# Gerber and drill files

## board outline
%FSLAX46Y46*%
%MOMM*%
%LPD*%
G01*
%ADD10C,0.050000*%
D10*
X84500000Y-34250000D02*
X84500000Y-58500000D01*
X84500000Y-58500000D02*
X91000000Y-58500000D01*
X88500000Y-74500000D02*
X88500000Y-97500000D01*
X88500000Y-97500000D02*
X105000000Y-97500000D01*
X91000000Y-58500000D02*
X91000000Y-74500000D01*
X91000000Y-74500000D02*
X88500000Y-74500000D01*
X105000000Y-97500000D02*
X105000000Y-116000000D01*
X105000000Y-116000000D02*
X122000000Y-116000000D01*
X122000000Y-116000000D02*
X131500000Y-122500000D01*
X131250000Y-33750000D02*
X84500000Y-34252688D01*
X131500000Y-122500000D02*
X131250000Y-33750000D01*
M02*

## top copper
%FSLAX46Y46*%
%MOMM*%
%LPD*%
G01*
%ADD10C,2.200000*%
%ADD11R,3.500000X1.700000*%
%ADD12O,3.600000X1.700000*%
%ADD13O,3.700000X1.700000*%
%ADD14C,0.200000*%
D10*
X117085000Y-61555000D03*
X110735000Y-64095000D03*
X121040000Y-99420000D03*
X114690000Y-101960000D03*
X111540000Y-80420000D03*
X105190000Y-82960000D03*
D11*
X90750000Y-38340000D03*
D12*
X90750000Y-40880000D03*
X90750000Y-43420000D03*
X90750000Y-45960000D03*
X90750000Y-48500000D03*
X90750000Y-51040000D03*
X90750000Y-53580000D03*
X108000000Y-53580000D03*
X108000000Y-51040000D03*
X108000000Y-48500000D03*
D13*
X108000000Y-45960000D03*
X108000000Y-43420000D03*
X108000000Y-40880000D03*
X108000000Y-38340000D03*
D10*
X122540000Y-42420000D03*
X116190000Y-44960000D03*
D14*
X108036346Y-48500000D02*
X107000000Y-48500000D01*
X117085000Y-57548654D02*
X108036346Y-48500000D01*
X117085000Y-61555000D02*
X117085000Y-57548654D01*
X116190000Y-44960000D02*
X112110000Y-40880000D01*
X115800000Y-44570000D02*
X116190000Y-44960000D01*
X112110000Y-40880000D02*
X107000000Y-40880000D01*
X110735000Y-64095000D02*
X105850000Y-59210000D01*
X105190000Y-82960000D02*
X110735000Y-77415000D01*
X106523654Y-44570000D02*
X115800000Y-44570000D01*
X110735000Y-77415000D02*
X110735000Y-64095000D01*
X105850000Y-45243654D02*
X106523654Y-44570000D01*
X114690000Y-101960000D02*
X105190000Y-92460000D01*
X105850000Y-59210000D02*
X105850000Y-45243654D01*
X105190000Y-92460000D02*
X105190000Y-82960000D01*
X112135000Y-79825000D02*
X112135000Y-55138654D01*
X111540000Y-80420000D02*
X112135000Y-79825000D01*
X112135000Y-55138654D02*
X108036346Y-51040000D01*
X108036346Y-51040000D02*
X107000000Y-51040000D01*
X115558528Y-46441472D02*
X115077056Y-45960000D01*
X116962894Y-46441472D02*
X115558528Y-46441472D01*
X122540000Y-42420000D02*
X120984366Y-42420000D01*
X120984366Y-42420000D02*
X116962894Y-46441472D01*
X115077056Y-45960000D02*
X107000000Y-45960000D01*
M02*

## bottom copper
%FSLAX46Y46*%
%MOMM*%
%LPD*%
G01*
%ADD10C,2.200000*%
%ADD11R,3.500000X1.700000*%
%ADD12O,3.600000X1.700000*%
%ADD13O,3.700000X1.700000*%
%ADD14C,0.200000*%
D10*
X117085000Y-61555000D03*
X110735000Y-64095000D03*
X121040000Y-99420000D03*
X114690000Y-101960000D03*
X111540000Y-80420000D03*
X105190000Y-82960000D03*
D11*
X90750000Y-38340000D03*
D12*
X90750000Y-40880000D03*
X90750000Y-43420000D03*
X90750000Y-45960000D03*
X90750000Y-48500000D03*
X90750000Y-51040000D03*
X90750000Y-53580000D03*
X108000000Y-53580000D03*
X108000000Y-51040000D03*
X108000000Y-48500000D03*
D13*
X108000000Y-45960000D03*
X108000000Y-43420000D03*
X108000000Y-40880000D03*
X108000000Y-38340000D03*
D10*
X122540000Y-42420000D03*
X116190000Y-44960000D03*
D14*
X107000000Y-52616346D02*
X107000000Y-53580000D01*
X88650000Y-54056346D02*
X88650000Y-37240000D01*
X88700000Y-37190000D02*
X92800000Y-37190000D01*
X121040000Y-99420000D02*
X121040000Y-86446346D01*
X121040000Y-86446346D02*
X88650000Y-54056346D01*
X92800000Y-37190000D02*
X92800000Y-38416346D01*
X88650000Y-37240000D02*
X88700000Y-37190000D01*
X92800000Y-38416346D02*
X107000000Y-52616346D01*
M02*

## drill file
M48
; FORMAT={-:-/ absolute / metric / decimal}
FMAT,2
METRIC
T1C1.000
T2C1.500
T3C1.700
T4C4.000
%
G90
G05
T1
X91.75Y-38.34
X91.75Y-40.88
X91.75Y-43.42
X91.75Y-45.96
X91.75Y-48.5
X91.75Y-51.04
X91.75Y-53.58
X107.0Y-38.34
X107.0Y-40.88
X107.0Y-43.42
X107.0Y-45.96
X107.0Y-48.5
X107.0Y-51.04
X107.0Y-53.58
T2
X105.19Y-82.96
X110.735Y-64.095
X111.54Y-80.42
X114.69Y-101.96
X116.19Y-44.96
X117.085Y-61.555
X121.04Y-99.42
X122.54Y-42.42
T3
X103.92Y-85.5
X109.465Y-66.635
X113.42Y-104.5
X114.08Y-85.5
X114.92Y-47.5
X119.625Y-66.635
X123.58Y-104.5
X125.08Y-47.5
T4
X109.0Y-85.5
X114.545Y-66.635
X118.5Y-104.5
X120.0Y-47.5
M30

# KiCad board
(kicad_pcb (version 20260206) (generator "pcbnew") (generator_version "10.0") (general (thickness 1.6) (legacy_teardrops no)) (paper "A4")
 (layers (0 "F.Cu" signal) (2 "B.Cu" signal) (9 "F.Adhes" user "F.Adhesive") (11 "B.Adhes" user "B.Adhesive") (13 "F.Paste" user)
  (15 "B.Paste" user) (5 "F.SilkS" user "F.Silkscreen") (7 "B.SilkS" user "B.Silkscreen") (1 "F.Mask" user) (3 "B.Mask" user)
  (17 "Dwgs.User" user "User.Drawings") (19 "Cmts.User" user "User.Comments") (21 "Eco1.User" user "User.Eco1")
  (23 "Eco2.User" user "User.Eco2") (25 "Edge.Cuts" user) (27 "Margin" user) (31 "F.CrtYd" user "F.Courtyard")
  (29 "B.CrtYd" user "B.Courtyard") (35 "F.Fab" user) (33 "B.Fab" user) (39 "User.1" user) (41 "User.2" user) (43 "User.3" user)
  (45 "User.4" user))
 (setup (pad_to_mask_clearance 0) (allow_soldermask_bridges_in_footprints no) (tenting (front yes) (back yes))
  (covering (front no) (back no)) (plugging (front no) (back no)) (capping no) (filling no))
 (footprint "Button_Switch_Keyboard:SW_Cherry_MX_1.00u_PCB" (layer "F.Cu") (at 117.085 61.555)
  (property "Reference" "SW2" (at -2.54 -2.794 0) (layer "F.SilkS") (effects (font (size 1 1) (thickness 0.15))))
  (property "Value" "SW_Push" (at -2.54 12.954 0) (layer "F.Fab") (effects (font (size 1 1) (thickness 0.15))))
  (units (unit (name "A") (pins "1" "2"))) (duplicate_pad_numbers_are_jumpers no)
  (pad "" np_thru_hole circle (at -7.62 5.08) (size 1.7 1.7) (drill 1.7) (layers "*.Cu" "*.Mask"))
  (pad "" np_thru_hole circle (at -2.54 5.08) (size 4 4) (drill 4) (layers "*.Cu" "*.Mask"))
  (pad "" np_thru_hole circle (at 2.54 5.08) (size 1.7 1.7) (drill 1.7) (layers "*.Cu" "*.Mask"))
  (pad "1" thru_hole circle (at 0 0) (size 2.2 2.2) (drill 1.5) (layers "*.Cu" "*.Mask") (remove_unused_layers no)
   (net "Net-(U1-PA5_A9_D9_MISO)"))
  (pad "2" thru_hole circle (at -6.35 2.54) (size 2.2 2.2) (drill 1.5) (layers "*.Cu" "*.Mask") (remove_unused_layers no) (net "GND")))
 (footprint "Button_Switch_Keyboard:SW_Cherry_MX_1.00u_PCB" (layer "F.Cu") (at 121.04 99.42)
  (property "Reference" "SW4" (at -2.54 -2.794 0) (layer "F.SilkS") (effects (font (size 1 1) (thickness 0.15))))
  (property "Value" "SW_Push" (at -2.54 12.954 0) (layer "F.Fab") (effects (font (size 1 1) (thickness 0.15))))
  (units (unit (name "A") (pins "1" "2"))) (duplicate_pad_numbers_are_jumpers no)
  (pad "" np_thru_hole circle (at -7.62 5.08) (size 1.7 1.7) (drill 1.7) (layers "*.Cu" "*.Mask"))
  (pad "" np_thru_hole circle (at -2.54 5.08) (size 4 4) (drill 4) (layers "*.Cu" "*.Mask"))
  (pad "" np_thru_hole circle (at 2.54 5.08) (size 1.7 1.7) (drill 1.7) (layers "*.Cu" "*.Mask"))
  (pad "1" thru_hole circle (at 0 0) (size 2.2 2.2) (drill 1.5) (layers "*.Cu" "*.Mask") (remove_unused_layers no)
   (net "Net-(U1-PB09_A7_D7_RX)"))
  (pad "2" thru_hole circle (at -6.35 2.54) (size 2.2 2.2) (drill 1.5) (layers "*.Cu" "*.Mask") (remove_unused_layers no) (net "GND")))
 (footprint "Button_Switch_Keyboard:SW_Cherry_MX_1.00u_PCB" (layer "F.Cu") (at 111.54 80.42)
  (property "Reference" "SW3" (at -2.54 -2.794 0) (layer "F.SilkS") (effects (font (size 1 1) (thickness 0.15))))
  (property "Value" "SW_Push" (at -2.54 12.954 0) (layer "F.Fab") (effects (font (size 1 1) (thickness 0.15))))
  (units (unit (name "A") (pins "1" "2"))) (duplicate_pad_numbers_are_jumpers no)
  (pad "" np_thru_hole circle (at -7.62 5.08) (size 1.7 1.7) (drill 1.7) (layers "*.Cu" "*.Mask"))
  (pad "" np_thru_hole circle (at -2.54 5.08) (size 4 4) (drill 4) (layers "*.Cu" "*.Mask"))
  (pad "" np_thru_hole circle (at 2.54 5.08) (size 1.7 1.7) (drill 1.7) (layers "*.Cu" "*.Mask"))
  (pad "1" thru_hole circle (at 0 0) (size 2.2 2.2) (drill 1.5) (layers "*.Cu" "*.Mask") (remove_unused_layers no)
   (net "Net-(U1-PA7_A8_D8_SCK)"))
  (pad "2" thru_hole circle (at -6.35 2.54) (size 2.2 2.2) (drill 1.5) (layers "*.Cu" "*.Mask") (remove_unused_layers no) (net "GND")))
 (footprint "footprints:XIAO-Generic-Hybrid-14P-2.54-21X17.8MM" (layer "F.Cu") (at 99.375 45.96)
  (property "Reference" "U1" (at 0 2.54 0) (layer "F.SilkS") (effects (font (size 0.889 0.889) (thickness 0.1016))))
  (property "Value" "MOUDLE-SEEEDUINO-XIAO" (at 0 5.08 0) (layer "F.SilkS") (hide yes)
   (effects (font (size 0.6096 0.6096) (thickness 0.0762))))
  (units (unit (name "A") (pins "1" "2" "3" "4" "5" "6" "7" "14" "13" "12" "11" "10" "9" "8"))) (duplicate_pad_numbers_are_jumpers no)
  (pad "1" thru_hole rect (at -7.625 -7.62) (size 3.5 1.7) (drill 1 (offset -1 0)) (layers "*.Cu" "*.Mask") (remove_unused_layers no)
   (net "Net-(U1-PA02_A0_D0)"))
  (pad "2" thru_hole oval (at -7.625 -5.08) (size 3.6 1.7) (drill 1 (offset -1 0)) (layers "*.Cu" "*.Mask") (remove_unused_layers no)
   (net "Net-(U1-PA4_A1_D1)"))
  (pad "3" thru_hole oval (at -7.625 -2.54) (size 3.6 1.7) (drill 1 (offset -1 0)) (layers "*.Cu" "*.Mask") (remove_unused_layers no)
   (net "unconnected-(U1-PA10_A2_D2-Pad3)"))
  (pad "4" thru_hole oval (at -7.625 0) (size 3.6 1.7) (drill 1 (offset -1 0)) (layers "*.Cu" "*.Mask") (remove_unused_layers no)
   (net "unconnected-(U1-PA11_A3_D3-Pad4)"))
  (pad "5" thru_hole oval (at -7.625 2.54) (size 3.6 1.7) (drill 1 (offset -1 0)) (layers "*.Cu" "*.Mask") (remove_unused_layers no)
   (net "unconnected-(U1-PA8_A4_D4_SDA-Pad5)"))
  (pad "6" thru_hole oval (at -7.625 5.08 180) (size 3.6 1.7) (drill 1 (offset 1 0)) (layers "*.Cu" "*.Mask") (remove_unused_layers no)
   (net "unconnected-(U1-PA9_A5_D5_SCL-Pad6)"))
  (pad "7" thru_hole oval (at -7.625 7.62) (size 3.6 1.7) (drill 1 (offset -1 0)) (layers "*.Cu" "*.Mask") (remove_unused_layers no)
   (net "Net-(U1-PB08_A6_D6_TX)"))
  (pad "8" thru_hole oval (at 7.625 7.62) (size 3.6 1.7) (drill 1 (offset 1 0)) (layers "*.Cu" "*.Mask") (remove_unused_layers no)
   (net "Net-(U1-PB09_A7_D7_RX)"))
  (pad "9" thru_hole oval (at 7.625 5.08) (size 3.6 1.7) (drill 1 (offset 1 0)) (layers "*.Cu" "*.Mask") (remove_unused_layers no)
   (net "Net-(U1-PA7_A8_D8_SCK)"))
  (pad "10" thru_hole oval (at 7.625 2.54) (size 3.6 1.7) (drill 1 (offset 1 0)) (layers "*.Cu" "*.Mask") (remove_unused_layers no)
   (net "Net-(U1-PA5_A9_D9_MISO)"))
  (pad "11" thru_hole oval (at 7.625 0) (size 3.7 1.7) (drill 1 (offset 1 0)) (layers "*.Cu" "*.Mask") (remove_unused_layers no)
   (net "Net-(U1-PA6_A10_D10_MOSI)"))
  (pad "12" thru_hole oval (at 7.625 -2.54) (size 3.7 1.7) (drill 1 (offset 1 0)) (layers "*.Cu" "*.Mask") (remove_unused_layers no)
   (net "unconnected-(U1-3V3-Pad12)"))
  (pad "13" thru_hole oval (at 7.625 -5.08) (size 3.7 1.7) (drill 1 (offset 1 0)) (layers "*.Cu" "*.Mask") (remove_unused_layers no)
   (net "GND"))
  (pad "14" thru_hole oval (at 7.625 -7.62) (size 3.7 1.7) (drill 1 (offset 1 0)) (layers "*.Cu" "*.Mask") (remove_unused_layers no)
   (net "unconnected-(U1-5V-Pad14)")))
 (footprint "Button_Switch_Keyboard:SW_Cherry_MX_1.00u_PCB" (layer "F.Cu") (at 122.54 42.42)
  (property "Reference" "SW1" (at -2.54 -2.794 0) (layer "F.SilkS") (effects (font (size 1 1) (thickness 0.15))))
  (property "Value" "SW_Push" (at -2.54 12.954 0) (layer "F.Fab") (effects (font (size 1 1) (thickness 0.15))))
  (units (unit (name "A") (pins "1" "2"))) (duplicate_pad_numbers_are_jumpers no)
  (pad "" np_thru_hole circle (at -7.62 5.08) (size 1.7 1.7) (drill 1.7) (layers "*.Cu" "*.Mask"))
  (pad "" np_thru_hole circle (at -2.54 5.08) (size 4 4) (drill 4) (layers "*.Cu" "*.Mask"))
  (pad "" np_thru_hole circle (at 2.54 5.08) (size 1.7 1.7) (drill 1.7) (layers "*.Cu" "*.Mask"))
  (pad "1" thru_hole circle (at 0 0) (size 2.2 2.2) (drill 1.5) (layers "*.Cu" "*.Mask") (remove_unused_layers no)
   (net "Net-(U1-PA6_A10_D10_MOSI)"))
  (pad "2" thru_hole circle (at -6.35 2.54) (size 2.2 2.2) (drill 1.5) (layers "*.Cu" "*.Mask") (remove_unused_layers no) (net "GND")))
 (gr_line (start 84.5 34.25) (end 84.5 58.5) (stroke (width 0.05) (type default)) (layer "Edge.Cuts"))
 (gr_line (start 84.5 58.5) (end 91 58.5) (stroke (width 0.05) (type default)) (layer "Edge.Cuts"))
 (gr_line (start 88.5 74.5) (end 88.5 97.5) (stroke (width 0.05) (type default)) (layer "Edge.Cuts"))
 (gr_line (start 88.5 97.5) (end 105 97.5) (stroke (width 0.05) (type default)) (layer "Edge.Cuts"))
 (gr_line (start 91 58.5) (end 91 74.5) (stroke (width 0.05) (type default)) (layer "Edge.Cuts"))
 (gr_line (start 91 74.5) (end 88.5 74.5) (stroke (width 0.05) (type default)) (layer "Edge.Cuts"))
 (gr_line (start 105 97.5) (end 105 116) (stroke (width 0.05) (type default)) (layer "Edge.Cuts"))
 (gr_line (start 105 116) (end 122 116) (stroke (width 0.05) (type default)) (layer "Edge.Cuts"))
 (gr_line (start 122 116) (end 131.5 122.5) (stroke (width 0.05) (type default)) (layer "Edge.Cuts"))
 (gr_line (start 131.25 33.75) (end 84.5 34.252688) (stroke (width 0.05) (type default)) (layer "Edge.Cuts"))
 (gr_line (start 131.5 122.5) (end 131.25 33.75) (stroke (width 0.05) (type default)) (layer "Edge.Cuts"))
 (segment (start 108.036346 48.5) (end 107 48.5) (width 0.2) (layer "F.Cu") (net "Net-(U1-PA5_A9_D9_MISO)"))
 (segment (start 117.085 57.548654) (end 108.036346 48.5) (width 0.2) (layer "F.Cu") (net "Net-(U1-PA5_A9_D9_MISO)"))
 (segment (start 117.085 61.555) (end 117.085 57.548654) (width 0.2) (layer "F.Cu") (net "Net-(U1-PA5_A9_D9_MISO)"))
 (segment (start 116.19 44.96) (end 112.11 40.88) (width 0.2) (layer "F.Cu") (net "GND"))
 (segment (start 115.8 44.57) (end 116.19 44.96) (width 0.2) (layer "F.Cu") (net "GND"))
 (segment (start 112.11 40.88) (end 107 40.88) (width 0.2) (layer "F.Cu") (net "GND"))
 (segment (start 110.735 64.095) (end 105.85 59.21) (width 0.2) (layer "F.Cu") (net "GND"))
 (segment (start 105.19 82.96) (end 110.735 77.415) (width 0.2) (layer "F.Cu") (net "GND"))
 (segment (start 106.523654 44.57) (end 115.8 44.57) (width 0.2) (layer "F.Cu") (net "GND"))
 (segment (start 110.735 77.415) (end 110.735 64.095) (width 0.2) (layer "F.Cu") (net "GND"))
 (segment (start 105.85 45.243654) (end 106.523654 44.57) (width 0.2) (layer "F.Cu") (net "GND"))
 (segment (start 114.69 101.96) (end 105.19 92.46) (width 0.2) (layer "F.Cu") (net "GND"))
 (segment (start 105.85 59.21) (end 105.85 45.243654) (width 0.2) (layer "F.Cu") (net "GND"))
 (segment (start 105.19 92.46) (end 105.19 82.96) (width 0.2) (layer "F.Cu") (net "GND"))
 (segment (start 107 52.616346) (end 107 53.58) (width 0.2) (layer "B.Cu") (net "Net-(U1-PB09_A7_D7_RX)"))
 (segment (start 88.65 54.056346) (end 88.65 37.24) (width 0.2) (layer "B.Cu") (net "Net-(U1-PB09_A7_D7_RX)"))
 (segment (start 88.7 37.19) (end 92.8 37.19) (width 0.2) (layer "B.Cu") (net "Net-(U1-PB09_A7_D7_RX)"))
 (segment (start 121.04 99.42) (end 121.04 86.446346) (width 0.2) (layer "B.Cu") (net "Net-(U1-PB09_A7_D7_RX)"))
 (segment (start 121.04 86.446346) (end 88.65 54.056346) (width 0.2) (layer "B.Cu") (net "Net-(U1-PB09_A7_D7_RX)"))
 (segment (start 92.8 37.19) (end 92.8 38.416346) (width 0.2) (layer "B.Cu") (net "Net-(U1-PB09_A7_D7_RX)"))
 (segment (start 88.65 37.24) (end 88.7 37.19) (width 0.2) (layer "B.Cu") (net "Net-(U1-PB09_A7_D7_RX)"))
 (segment (start 92.8 38.416346) (end 107 52.616346) (width 0.2) (layer "B.Cu") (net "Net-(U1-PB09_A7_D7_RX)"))
 (segment (start 112.135 79.825) (end 112.135 55.138654) (width 0.2) (layer "F.Cu") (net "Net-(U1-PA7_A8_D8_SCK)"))
 (segment (start 111.54 80.42) (end 112.135 79.825) (width 0.2) (layer "F.Cu") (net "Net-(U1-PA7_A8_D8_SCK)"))
 (segment (start 112.135 55.138654) (end 108.036346 51.04) (width 0.2) (layer "F.Cu") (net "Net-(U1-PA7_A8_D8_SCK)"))
 (segment (start 108.036346 51.04) (end 107 51.04) (width 0.2) (layer "F.Cu") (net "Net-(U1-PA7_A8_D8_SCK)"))
 (segment (start 115.558528 46.441472) (end 115.077056 45.96) (width 0.2) (layer "F.Cu") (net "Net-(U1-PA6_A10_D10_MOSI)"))
 (segment (start 116.962894 46.441472) (end 115.558528 46.441472) (width 0.2) (layer "F.Cu") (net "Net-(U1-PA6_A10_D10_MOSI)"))
 (segment (start 122.54 42.42) (end 120.984366 42.42) (width 0.2) (layer "F.Cu") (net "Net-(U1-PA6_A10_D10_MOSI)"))
 (segment (start 120.984366 42.42) (end 116.962894 46.441472) (width 0.2) (layer "F.Cu") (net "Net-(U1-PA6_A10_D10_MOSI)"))
 (segment (start 115.077056 45.96) (end 107 45.96) (width 0.2) (layer "F.Cu") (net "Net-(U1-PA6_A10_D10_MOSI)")))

